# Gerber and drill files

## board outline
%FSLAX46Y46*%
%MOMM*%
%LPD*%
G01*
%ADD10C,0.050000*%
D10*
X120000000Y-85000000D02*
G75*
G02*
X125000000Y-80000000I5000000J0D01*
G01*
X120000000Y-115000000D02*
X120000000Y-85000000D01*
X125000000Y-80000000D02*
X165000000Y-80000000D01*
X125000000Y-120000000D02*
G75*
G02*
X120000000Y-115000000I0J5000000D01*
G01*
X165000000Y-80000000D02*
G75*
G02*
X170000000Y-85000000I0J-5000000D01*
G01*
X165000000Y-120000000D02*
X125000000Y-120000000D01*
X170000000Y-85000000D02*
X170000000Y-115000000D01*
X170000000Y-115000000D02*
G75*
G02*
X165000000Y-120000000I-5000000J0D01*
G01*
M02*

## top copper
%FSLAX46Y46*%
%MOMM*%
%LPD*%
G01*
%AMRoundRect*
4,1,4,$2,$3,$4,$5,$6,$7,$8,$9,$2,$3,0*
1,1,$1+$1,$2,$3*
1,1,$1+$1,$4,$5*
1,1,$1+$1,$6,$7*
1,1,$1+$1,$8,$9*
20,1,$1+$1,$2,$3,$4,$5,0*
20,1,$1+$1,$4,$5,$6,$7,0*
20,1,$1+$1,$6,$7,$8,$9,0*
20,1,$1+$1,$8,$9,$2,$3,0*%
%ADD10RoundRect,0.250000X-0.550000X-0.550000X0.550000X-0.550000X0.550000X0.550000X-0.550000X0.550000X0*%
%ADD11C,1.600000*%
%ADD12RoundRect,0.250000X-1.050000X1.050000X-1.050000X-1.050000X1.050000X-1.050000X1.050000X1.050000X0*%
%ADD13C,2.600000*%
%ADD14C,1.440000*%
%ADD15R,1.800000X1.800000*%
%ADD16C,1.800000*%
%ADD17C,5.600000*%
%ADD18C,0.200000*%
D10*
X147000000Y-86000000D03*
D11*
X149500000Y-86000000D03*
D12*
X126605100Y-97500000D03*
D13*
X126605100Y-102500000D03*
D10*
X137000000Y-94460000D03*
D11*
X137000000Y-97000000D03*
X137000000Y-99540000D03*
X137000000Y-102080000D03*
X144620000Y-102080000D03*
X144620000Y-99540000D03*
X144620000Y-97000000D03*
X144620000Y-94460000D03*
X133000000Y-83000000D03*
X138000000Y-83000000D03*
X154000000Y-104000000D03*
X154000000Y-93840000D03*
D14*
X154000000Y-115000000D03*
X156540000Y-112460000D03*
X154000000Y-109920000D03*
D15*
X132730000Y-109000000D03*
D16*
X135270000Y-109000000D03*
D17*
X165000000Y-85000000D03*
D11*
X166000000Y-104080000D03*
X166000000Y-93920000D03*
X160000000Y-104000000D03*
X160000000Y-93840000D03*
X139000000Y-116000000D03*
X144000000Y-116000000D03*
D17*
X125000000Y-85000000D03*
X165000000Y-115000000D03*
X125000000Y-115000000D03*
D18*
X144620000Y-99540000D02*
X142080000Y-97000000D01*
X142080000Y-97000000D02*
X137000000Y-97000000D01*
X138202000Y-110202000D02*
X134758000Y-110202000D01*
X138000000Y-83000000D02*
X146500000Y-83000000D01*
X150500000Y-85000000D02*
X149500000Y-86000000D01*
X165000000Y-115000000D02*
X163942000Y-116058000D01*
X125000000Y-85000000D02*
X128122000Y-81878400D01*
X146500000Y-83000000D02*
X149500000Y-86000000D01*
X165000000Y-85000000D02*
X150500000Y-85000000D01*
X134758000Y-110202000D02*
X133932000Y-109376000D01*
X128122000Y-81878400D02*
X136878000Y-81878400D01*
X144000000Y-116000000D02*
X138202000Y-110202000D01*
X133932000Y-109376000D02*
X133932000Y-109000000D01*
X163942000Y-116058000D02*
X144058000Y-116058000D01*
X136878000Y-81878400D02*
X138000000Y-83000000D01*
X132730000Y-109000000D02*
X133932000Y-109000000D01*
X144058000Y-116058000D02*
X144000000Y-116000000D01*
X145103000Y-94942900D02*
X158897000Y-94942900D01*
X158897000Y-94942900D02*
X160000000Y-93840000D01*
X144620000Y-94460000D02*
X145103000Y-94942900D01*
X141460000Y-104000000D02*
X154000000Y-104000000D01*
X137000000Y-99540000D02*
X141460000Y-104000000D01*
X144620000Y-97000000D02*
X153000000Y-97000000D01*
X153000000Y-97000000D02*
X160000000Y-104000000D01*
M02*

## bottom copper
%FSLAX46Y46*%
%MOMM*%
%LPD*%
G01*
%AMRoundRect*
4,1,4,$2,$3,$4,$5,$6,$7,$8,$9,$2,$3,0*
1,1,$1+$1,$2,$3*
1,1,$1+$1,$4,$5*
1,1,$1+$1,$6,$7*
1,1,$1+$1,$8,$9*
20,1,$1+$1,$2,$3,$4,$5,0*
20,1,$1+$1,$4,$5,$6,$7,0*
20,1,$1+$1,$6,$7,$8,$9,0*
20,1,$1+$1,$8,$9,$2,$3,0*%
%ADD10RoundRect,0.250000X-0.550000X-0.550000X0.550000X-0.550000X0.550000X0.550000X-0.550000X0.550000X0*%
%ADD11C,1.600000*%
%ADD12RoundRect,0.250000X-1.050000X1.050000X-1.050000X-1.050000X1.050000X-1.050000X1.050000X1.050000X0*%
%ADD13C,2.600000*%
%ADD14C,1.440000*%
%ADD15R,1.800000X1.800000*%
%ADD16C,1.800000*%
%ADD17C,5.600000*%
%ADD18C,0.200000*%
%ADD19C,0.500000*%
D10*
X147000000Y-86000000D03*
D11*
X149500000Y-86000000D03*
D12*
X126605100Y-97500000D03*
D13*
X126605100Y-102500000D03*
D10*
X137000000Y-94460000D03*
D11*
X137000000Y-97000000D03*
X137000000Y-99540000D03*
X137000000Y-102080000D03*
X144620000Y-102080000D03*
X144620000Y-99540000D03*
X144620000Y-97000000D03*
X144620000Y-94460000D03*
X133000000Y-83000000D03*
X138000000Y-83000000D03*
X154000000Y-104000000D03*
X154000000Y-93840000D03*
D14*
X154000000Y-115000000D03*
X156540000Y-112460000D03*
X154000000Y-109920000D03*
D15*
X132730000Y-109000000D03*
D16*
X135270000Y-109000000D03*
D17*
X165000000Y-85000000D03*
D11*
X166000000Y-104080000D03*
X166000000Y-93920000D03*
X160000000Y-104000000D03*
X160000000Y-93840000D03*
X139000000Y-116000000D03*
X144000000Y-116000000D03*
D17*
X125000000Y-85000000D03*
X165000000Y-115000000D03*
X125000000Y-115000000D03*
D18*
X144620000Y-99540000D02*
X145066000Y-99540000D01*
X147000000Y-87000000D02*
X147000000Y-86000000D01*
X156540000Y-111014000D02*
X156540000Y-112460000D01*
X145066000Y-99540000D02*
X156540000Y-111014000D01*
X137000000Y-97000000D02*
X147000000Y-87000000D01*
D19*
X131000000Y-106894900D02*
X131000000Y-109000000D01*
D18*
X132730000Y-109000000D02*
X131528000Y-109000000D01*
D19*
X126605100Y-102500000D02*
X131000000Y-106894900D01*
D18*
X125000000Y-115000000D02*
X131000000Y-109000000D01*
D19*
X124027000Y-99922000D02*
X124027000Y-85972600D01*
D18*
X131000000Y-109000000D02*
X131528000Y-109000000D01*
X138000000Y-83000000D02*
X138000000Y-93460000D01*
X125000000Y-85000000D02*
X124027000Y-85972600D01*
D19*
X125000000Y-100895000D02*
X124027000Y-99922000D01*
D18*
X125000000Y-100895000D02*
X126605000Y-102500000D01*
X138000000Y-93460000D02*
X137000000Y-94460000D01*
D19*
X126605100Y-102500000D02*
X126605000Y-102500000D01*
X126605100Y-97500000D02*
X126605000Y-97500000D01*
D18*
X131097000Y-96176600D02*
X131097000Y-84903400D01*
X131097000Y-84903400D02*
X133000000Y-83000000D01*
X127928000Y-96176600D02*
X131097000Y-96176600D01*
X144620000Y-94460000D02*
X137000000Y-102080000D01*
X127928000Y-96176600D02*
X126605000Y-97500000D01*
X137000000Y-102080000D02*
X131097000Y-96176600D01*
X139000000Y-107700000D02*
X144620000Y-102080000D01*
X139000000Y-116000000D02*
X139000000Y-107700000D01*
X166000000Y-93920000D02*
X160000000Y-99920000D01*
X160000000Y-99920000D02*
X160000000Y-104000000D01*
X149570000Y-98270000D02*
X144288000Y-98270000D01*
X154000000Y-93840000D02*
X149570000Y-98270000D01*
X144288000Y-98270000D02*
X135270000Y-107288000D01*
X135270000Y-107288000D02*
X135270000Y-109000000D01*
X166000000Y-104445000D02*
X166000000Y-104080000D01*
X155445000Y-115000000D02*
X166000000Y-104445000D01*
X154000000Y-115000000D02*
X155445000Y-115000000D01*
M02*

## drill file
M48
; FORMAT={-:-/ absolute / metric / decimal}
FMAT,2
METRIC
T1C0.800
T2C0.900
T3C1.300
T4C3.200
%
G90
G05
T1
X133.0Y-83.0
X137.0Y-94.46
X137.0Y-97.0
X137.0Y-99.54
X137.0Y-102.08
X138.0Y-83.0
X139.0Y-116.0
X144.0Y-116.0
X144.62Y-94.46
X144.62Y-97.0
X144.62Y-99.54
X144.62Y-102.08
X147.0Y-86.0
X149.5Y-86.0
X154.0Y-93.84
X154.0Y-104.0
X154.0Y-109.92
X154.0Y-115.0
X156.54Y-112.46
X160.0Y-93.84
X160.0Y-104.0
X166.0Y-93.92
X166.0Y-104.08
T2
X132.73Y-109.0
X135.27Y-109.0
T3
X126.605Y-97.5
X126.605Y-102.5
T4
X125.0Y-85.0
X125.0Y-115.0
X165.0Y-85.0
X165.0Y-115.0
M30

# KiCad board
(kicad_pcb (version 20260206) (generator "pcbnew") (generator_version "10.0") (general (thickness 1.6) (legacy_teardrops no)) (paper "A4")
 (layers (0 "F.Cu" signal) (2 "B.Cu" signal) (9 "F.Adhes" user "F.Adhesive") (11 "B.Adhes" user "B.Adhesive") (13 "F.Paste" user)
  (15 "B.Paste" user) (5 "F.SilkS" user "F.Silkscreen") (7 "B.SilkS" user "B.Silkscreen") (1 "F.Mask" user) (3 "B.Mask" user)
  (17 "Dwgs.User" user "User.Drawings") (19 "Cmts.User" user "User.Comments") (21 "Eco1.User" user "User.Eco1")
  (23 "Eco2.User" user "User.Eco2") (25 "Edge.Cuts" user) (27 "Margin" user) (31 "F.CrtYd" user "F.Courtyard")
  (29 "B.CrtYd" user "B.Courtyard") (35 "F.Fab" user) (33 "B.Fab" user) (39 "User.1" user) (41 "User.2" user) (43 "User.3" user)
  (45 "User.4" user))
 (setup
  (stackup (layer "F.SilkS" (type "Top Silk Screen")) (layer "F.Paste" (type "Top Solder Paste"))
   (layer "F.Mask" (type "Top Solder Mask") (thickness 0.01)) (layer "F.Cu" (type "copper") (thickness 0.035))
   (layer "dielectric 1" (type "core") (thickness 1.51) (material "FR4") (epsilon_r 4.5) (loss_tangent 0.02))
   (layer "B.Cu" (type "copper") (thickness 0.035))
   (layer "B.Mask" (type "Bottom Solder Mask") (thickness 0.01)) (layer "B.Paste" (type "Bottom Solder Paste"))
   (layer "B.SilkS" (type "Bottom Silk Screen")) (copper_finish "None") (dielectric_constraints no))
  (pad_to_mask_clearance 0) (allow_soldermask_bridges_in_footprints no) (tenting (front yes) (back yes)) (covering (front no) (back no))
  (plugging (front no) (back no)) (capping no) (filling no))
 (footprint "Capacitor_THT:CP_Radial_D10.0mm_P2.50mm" (layer "F.Cu") (at 147 86)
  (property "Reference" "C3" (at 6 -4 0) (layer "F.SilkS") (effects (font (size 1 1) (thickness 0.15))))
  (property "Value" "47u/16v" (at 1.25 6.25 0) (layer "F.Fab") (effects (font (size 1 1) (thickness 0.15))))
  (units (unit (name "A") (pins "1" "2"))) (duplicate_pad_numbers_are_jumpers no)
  (pad "1" thru_hole roundrect (at 0 0) (size 1.6 1.6) (drill 0.8) (layers "*.Cu" "*.Mask") (remove_unused_layers no)
   (roundrect_rratio 0.15625) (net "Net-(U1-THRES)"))
  (pad "2" thru_hole circle (at 2.5 0) (size 1.6 1.6) (drill 0.8) (layers "*.Cu" "*.Mask") (remove_unused_layers no) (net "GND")))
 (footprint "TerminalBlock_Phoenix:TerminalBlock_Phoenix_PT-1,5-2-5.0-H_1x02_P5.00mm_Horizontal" (layer "F.Cu") (at 126.6051 97.5 -90)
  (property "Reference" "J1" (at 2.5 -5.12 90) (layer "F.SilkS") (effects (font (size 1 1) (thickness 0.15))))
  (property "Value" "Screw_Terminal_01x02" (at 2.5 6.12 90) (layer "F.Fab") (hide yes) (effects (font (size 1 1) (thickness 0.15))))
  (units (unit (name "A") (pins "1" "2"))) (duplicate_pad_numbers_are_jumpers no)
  (pad "1" thru_hole roundrect (at 0 0 270) (size 2.6 2.6) (drill 1.3) (layers "*.Cu" "*.Mask") (remove_unused_layers no)
   (roundrect_rratio 0.096154) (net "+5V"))
  (pad "2" thru_hole circle (at 5 0 270) (size 2.6 2.6) (drill 1.3) (layers "*.Cu" "*.Mask") (remove_unused_layers no) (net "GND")))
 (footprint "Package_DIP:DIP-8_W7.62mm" (layer "F.Cu") (at 137 94.46)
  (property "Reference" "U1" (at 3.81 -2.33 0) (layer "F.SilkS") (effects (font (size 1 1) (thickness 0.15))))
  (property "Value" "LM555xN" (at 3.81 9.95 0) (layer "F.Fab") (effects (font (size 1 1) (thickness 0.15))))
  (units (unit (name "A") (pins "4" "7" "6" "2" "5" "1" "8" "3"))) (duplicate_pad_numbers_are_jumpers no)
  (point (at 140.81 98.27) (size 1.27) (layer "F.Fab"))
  (pad "1" thru_hole roundrect (at 0 0) (size 1.6 1.6) (drill 0.8) (layers "*.Cu" "*.Mask") (remove_unused_layers no)
   (roundrect_rratio 0.15625) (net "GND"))
  (pad "2" thru_hole circle (at 0 2.54) (size 1.6 1.6) (drill 0.8) (layers "*.Cu" "*.Mask") (remove_unused_layers no) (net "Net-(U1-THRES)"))
  (pad "3" thru_hole circle (at 0 5.08) (size 1.6 1.6) (drill 0.8) (layers "*.Cu" "*.Mask") (remove_unused_layers no) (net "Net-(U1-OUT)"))
  (pad "4" thru_hole circle (at 0 7.62) (size 1.6 1.6) (drill 0.8) (layers "*.Cu" "*.Mask") (remove_unused_layers no) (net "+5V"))
  (pad "5" thru_hole circle (at 7.62 7.62) (size 1.6 1.6) (drill 0.8) (layers "*.Cu" "*.Mask") (remove_unused_layers no)
   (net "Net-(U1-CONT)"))
  (pad "6" thru_hole circle (at 7.62 5.08) (size 1.6 1.6) (drill 0.8) (layers "*.Cu" "*.Mask") (remove_unused_layers no)
   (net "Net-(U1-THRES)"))
  (pad "7" thru_hole circle (at 7.62 2.54) (size 1.6 1.6) (drill 0.8) (layers "*.Cu" "*.Mask") (remove_unused_layers no)
   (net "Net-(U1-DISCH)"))
  (pad "8" thru_hole circle (at 7.62 0) (size 1.6 1.6) (drill 0.8) (layers "*.Cu" "*.Mask") (remove_unused_layers no) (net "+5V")))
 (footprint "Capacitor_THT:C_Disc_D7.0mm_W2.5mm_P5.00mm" (layer "F.Cu") (at 133 83)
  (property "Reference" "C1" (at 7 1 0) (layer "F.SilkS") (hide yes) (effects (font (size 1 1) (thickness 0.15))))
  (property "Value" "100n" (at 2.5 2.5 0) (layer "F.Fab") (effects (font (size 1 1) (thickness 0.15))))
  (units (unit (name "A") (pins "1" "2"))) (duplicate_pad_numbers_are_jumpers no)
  (pad "1" thru_hole circle (at 0 0) (size 1.6 1.6) (drill 0.8) (layers "*.Cu" "*.Mask") (remove_unused_layers no) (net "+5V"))
  (pad "2" thru_hole circle (at 5 0) (size 1.6 1.6) (drill 0.8) (layers "*.Cu" "*.Mask") (remove_unused_layers no) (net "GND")))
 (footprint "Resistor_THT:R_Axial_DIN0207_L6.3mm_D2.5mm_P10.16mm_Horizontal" (layer "F.Cu") (at 154 104 90)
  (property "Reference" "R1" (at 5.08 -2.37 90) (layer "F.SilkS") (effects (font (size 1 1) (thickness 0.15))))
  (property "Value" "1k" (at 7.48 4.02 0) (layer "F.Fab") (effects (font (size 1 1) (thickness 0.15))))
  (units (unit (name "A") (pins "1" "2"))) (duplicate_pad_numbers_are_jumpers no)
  (pad "1" thru_hole circle (at 0 0 90) (size 1.6 1.6) (drill 0.8) (layers "*.Cu" "*.Mask") (remove_unused_layers no) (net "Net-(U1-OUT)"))
  (pad "2" thru_hole circle (at 10.16 0 90) (size 1.6 1.6) (drill 0.8) (layers "*.Cu" "*.Mask") (remove_unused_layers no) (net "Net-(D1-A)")))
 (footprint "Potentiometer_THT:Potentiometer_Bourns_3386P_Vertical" (layer "F.Cu") (at 154 115)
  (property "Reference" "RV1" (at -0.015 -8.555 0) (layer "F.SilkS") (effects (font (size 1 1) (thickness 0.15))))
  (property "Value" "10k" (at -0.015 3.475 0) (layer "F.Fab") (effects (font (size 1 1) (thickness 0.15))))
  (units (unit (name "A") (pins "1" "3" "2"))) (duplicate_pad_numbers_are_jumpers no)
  (pad "1" thru_hole circle (at 0 0) (size 1.44 1.44) (drill 0.8) (layers "*.Cu" "*.Mask") (remove_unused_layers no) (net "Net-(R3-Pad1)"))
  (pad "2" thru_hole circle (at 2.54 -2.54) (size 1.44 1.44) (drill 0.8) (layers "*.Cu" "*.Mask") (remove_unused_layers no)
   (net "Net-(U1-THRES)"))
  (pad "3" thru_hole circle (at 0 -5.08) (size 1.44 1.44) (drill 0.8) (layers "*.Cu" "*.Mask") (remove_unused_layers no)
   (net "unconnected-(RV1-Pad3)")))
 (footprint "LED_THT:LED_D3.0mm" (layer "F.Cu") (at 132.73 109)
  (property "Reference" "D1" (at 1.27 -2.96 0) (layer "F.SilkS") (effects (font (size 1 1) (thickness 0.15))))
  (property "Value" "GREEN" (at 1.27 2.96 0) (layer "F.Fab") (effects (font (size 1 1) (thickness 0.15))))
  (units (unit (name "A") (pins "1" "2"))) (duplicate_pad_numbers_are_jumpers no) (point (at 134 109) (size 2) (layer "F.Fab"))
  (pad "1" thru_hole rect (at 0 0) (size 1.8 1.8) (drill 0.9) (layers "*.Cu" "*.Mask") (remove_unused_layers no) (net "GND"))
  (pad "2" thru_hole circle (at 2.54 0) (size 1.8 1.8) (drill 0.9) (layers "*.Cu" "*.Mask") (remove_unused_layers no) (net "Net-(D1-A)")))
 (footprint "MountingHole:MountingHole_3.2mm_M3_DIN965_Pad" (layer "F.Cu") (at 165 85)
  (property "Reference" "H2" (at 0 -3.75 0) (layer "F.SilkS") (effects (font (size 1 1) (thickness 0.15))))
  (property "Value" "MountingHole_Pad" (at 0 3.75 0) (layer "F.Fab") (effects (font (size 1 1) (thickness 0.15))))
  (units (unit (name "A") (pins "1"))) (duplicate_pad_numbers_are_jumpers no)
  (pad "1" thru_hole circle (at 0 0) (size 5.6 5.6) (drill 3.2) (layers "*.Cu" "*.Mask") (remove_unused_layers no) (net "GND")
   (zone_connect 2)))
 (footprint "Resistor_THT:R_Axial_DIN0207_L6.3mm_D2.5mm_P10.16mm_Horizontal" (layer "F.Cu") (at 166 104.08 90)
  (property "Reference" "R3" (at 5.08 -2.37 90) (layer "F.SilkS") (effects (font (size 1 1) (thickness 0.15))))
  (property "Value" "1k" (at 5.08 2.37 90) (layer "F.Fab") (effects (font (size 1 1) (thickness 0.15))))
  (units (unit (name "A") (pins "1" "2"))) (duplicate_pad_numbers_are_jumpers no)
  (pad "1" thru_hole circle (at 0 0 90) (size 1.6 1.6) (drill 0.8) (layers "*.Cu" "*.Mask") (remove_unused_layers no) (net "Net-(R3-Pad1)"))
  (pad "2" thru_hole circle (at 10.16 0 90) (size 1.6 1.6) (drill 0.8) (layers "*.Cu" "*.Mask") (remove_unused_layers no)
   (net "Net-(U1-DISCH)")))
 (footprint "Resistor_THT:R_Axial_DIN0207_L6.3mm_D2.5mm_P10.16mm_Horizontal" (layer "F.Cu") (at 160 104 90)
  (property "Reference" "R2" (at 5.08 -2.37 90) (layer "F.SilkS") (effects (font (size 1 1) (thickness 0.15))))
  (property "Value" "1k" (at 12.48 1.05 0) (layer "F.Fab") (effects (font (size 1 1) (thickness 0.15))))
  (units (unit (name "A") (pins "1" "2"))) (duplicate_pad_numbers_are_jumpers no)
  (pad "1" thru_hole circle (at 0 0 90) (size 1.6 1.6) (drill 0.8) (layers "*.Cu" "*.Mask") (remove_unused_layers no) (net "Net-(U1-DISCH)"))
  (pad "2" thru_hole circle (at 10.16 0 90) (size 1.6 1.6) (drill 0.8) (layers "*.Cu" "*.Mask") (remove_unused_layers no) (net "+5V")))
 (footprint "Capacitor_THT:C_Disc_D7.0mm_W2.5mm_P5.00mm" (layer "F.Cu") (at 139 116)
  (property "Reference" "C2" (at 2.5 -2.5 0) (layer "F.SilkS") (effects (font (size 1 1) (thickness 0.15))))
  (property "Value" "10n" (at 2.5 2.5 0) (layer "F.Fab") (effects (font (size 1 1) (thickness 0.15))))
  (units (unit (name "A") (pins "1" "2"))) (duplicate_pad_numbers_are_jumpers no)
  (pad "1" thru_hole circle (at 0 0) (size 1.6 1.6) (drill 0.8) (layers "*.Cu" "*.Mask") (remove_unused_layers no) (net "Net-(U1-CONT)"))
  (pad "2" thru_hole circle (at 5 0) (size 1.6 1.6) (drill 0.8) (layers "*.Cu" "*.Mask") (remove_unused_layers no) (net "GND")))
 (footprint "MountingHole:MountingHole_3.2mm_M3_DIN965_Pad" (layer "F.Cu") (at 125 85)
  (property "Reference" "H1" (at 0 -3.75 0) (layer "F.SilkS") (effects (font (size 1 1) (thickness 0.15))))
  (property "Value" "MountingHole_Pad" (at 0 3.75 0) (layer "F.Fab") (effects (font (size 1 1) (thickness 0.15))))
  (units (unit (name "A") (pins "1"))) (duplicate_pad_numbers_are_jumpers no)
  (pad "1" thru_hole circle (at 0 0) (size 5.6 5.6) (drill 3.2) (layers "*.Cu" "*.Mask") (remove_unused_layers no) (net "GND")
   (zone_connect 2)))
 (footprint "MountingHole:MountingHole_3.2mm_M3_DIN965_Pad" (layer "F.Cu") (at 165 115)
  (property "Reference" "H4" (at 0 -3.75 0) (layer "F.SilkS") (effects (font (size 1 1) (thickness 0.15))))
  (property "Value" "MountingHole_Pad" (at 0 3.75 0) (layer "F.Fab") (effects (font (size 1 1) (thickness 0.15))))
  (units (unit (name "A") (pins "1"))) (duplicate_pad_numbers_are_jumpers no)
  (pad "1" thru_hole circle (at 0 0) (size 5.6 5.6) (drill 3.2) (layers "*.Cu" "*.Mask") (remove_unused_layers no) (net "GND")
   (zone_connect 2)))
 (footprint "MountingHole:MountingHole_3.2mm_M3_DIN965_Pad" (layer "F.Cu") (at 125 115)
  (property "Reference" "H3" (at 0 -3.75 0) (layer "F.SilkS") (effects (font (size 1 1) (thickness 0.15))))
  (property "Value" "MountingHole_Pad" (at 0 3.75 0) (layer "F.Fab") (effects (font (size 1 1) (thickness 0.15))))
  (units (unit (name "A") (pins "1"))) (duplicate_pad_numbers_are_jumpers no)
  (pad "1" thru_hole circle (at 0 0) (size 5.6 5.6) (drill 3.2) (layers "*.Cu" "*.Mask") (remove_unused_layers no) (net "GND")
   (zone_connect 2)))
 (gr_arc (start 120 85) (mid 121.464466 81.464466) (end 125 80) (stroke (width 0.05) (type default)) (layer "Edge.Cuts"))
 (gr_line (start 120 115) (end 120 85) (stroke (width 0.05) (type default)) (layer "Edge.Cuts"))
 (gr_line (start 125 80) (end 165 80) (stroke (width 0.05) (type default)) (layer "Edge.Cuts"))
 (gr_arc (start 125 120) (mid 121.464466 118.535534) (end 120 115) (stroke (width 0.05) (type default)) (layer "Edge.Cuts"))
 (gr_arc (start 165 80) (mid 168.535534 81.464466) (end 170 85) (stroke (width 0.05) (type default)) (layer "Edge.Cuts"))
 (gr_line (start 165 120) (end 125 120) (stroke (width 0.05) (type default)) (layer "Edge.Cuts"))
 (gr_line (start 170 85) (end 170 115) (stroke (width 0.05) (type default)) (layer "Edge.Cuts"))
 (gr_arc (start 170 115) (mid 168.535534 118.535534) (end 165 120) (stroke (width 0.05) (type default)) (layer "Edge.Cuts"))
 (segment (start 144.62 99.54) (end 142.08 97) (width 0.2) (layer "F.Cu") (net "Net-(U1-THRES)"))
 (segment (start 142.08 97) (end 137 97) (width 0.2) (layer "F.Cu") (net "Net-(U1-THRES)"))
 (segment (start 144.62 99.54) (end 145.066 99.54) (width 0.2) (layer "B.Cu") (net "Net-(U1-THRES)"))
 (segment (start 147 87) (end 147 86) (width 0.2) (layer "B.Cu") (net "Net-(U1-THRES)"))
 (segment (start 156.54 111.014) (end 156.54 112.46) (width 0.2) (layer "B.Cu") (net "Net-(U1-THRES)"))
 (segment (start 145.066 99.54) (end 156.54 111.014) (width 0.2) (layer "B.Cu") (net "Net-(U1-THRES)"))
 (segment (start 137 97) (end 147 87) (width 0.2) (layer "B.Cu") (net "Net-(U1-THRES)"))
 (segment (start 138.202 110.202) (end 134.758 110.202) (width 0.2) (layer "F.Cu") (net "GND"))
 (segment (start 138 83) (end 146.5 83) (width 0.2) (layer "F.Cu") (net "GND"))
 (segment (start 150.5 85) (end 149.5 86) (width 0.2) (layer "F.Cu") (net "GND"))
 (segment (start 165 115) (end 163.942 116.058) (width 0.2) (layer "F.Cu") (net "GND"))
 (segment (start 125 85) (end 128.122 81.8784) (width 0.2) (layer "F.Cu") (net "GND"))
 (segment (start 146.5 83) (end 149.5 86) (width 0.2) (layer "F.Cu") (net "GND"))
 (segment (start 165 85) (end 150.5 85) (width 0.2) (layer "F.Cu") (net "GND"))
 (segment (start 134.758 110.202) (end 133.932 109.376) (width 0.2) (layer "F.Cu") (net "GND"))
 (segment (start 128.122 81.8784) (end 136.878 81.8784) (width 0.2) (layer "F.Cu") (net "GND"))
 (segment (start 144 116) (end 138.202 110.202) (width 0.2) (layer "F.Cu") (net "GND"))
 (segment (start 133.932 109.376) (end 133.932 109) (width 0.2) (layer "F.Cu") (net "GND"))
 (segment (start 163.942 116.058) (end 144.058 116.058) (width 0.2) (layer "F.Cu") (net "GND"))
 (segment (start 136.878 81.8784) (end 138 83) (width 0.2) (layer "F.Cu") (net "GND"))
 (segment (start 132.73 109) (end 133.932 109) (width 0.2) (layer "F.Cu") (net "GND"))
 (segment (start 144.058 116.058) (end 144 116) (width 0.2) (layer "F.Cu") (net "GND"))
 (segment (start 131 106.8949) (end 131 109) (width 0.5) (layer "B.Cu") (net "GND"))
 (segment (start 132.73 109) (end 131.528 109) (width 0.2) (layer "B.Cu") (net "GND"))
 (segment (start 126.6051 102.5) (end 131 106.8949) (width 0.5) (layer "B.Cu") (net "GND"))
 (segment (start 125 115) (end 131 109) (width 0.2) (layer "B.Cu") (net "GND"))
 (segment (start 124.027 99.922) (end 124.027 85.9726) (width 0.5) (layer "B.Cu") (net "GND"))
 (segment (start 131 109) (end 131.528 109) (width 0.2) (layer "B.Cu") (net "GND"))
 (segment (start 138 83) (end 138 93.46) (width 0.2) (layer "B.Cu") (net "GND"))
 (segment (start 125 85) (end 124.027 85.9726) (width 0.2) (layer "B.Cu") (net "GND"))
 (segment (start 125 100.895) (end 124.027 99.922) (width 0.5) (layer "B.Cu") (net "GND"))
 (segment (start 125 100.895) (end 126.605 102.5) (width 0.2) (layer "B.Cu") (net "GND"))
 (segment (start 138 93.46) (end 137 94.46) (width 0.2) (layer "B.Cu") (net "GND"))
 (segment (start 126.6051 102.5) (end 126.605 102.5) (width 0.5) (layer "B.Cu") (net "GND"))
 (segment (start 145.103 94.9429) (end 158.897 94.9429) (width 0.2) (layer "F.Cu") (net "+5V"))
 (segment (start 158.897 94.9429) (end 160 93.84) (width 0.2) (layer "F.Cu") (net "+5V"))
 (segment (start 144.62 94.46) (end 145.103 94.9429) (width 0.2) (layer "F.Cu") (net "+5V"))
 (segment (start 126.6051 97.5) (end 126.605 97.5) (width 0.5) (layer "B.Cu") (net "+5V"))
 (segment (start 131.097 96.1766) (end 131.097 84.9034) (width 0.2) (layer "B.Cu") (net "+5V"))
 (segment (start 131.097 84.9034) (end 133 83) (width 0.2) (layer "B.Cu") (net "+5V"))
 (segment (start 127.928 96.1766) (end 131.097 96.1766) (width 0.2) (layer "B.Cu") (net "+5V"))
 (segment (start 144.62 94.46) (end 137 102.08) (width 0.2) (layer "B.Cu") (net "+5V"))
 (segment (start 127.928 96.1766) (end 126.605 97.5) (width 0.2) (layer "B.Cu") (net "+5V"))
 (segment (start 137 102.08) (end 131.097 96.1766) (width 0.2) (layer "B.Cu") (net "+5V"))
 (segment (start 141.46 104) (end 154 104) (width 0.2) (layer "F.Cu") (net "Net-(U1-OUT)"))
 (segment (start 137 99.54) (end 141.46 104) (width 0.2) (layer "F.Cu") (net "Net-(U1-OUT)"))
 (segment (start 139 107.7) (end 144.62 102.08) (width 0.2) (layer "B.Cu") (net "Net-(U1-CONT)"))
 (segment (start 139 116) (end 139 107.7) (width 0.2) (layer "B.Cu") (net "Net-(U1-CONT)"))
 (segment (start 144.62 97) (end 153 97) (width 0.2) (layer "F.Cu") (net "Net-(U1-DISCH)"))
 (segment (start 153 97) (end 160 104) (width 0.2) (layer "F.Cu") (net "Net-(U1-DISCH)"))
 (segment (start 166 93.92) (end 160 99.92) (width 0.2) (layer "B.Cu") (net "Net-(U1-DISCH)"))
 (segment (start 160 99.92) (end 160 104) (width 0.2) (layer "B.Cu") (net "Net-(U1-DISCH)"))
 (segment (start 149.57 98.27) (end 144.288 98.27) (width 0.2) (layer "B.Cu") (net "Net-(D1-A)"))
 (segment (start 154 93.84) (end 149.57 98.27) (width 0.2) (layer "B.Cu") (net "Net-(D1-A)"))
 (segment (start 144.288 98.27) (end 135.27 107.288) (width 0.2) (layer "B.Cu") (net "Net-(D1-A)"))
 (segment (start 135.27 107.288) (end 135.27 109) (width 0.2) (layer "B.Cu") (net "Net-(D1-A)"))
 (segment (start 166 104.445) (end 166 104.08) (width 0.2) (layer "B.Cu") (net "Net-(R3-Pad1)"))
 (segment (start 155.445 115) (end 166 104.445) (width 0.2) (layer "B.Cu") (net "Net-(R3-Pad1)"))
 (segment (start 154 115) (end 155.445 115) (width 0.2) (layer "B.Cu") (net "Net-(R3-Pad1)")))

